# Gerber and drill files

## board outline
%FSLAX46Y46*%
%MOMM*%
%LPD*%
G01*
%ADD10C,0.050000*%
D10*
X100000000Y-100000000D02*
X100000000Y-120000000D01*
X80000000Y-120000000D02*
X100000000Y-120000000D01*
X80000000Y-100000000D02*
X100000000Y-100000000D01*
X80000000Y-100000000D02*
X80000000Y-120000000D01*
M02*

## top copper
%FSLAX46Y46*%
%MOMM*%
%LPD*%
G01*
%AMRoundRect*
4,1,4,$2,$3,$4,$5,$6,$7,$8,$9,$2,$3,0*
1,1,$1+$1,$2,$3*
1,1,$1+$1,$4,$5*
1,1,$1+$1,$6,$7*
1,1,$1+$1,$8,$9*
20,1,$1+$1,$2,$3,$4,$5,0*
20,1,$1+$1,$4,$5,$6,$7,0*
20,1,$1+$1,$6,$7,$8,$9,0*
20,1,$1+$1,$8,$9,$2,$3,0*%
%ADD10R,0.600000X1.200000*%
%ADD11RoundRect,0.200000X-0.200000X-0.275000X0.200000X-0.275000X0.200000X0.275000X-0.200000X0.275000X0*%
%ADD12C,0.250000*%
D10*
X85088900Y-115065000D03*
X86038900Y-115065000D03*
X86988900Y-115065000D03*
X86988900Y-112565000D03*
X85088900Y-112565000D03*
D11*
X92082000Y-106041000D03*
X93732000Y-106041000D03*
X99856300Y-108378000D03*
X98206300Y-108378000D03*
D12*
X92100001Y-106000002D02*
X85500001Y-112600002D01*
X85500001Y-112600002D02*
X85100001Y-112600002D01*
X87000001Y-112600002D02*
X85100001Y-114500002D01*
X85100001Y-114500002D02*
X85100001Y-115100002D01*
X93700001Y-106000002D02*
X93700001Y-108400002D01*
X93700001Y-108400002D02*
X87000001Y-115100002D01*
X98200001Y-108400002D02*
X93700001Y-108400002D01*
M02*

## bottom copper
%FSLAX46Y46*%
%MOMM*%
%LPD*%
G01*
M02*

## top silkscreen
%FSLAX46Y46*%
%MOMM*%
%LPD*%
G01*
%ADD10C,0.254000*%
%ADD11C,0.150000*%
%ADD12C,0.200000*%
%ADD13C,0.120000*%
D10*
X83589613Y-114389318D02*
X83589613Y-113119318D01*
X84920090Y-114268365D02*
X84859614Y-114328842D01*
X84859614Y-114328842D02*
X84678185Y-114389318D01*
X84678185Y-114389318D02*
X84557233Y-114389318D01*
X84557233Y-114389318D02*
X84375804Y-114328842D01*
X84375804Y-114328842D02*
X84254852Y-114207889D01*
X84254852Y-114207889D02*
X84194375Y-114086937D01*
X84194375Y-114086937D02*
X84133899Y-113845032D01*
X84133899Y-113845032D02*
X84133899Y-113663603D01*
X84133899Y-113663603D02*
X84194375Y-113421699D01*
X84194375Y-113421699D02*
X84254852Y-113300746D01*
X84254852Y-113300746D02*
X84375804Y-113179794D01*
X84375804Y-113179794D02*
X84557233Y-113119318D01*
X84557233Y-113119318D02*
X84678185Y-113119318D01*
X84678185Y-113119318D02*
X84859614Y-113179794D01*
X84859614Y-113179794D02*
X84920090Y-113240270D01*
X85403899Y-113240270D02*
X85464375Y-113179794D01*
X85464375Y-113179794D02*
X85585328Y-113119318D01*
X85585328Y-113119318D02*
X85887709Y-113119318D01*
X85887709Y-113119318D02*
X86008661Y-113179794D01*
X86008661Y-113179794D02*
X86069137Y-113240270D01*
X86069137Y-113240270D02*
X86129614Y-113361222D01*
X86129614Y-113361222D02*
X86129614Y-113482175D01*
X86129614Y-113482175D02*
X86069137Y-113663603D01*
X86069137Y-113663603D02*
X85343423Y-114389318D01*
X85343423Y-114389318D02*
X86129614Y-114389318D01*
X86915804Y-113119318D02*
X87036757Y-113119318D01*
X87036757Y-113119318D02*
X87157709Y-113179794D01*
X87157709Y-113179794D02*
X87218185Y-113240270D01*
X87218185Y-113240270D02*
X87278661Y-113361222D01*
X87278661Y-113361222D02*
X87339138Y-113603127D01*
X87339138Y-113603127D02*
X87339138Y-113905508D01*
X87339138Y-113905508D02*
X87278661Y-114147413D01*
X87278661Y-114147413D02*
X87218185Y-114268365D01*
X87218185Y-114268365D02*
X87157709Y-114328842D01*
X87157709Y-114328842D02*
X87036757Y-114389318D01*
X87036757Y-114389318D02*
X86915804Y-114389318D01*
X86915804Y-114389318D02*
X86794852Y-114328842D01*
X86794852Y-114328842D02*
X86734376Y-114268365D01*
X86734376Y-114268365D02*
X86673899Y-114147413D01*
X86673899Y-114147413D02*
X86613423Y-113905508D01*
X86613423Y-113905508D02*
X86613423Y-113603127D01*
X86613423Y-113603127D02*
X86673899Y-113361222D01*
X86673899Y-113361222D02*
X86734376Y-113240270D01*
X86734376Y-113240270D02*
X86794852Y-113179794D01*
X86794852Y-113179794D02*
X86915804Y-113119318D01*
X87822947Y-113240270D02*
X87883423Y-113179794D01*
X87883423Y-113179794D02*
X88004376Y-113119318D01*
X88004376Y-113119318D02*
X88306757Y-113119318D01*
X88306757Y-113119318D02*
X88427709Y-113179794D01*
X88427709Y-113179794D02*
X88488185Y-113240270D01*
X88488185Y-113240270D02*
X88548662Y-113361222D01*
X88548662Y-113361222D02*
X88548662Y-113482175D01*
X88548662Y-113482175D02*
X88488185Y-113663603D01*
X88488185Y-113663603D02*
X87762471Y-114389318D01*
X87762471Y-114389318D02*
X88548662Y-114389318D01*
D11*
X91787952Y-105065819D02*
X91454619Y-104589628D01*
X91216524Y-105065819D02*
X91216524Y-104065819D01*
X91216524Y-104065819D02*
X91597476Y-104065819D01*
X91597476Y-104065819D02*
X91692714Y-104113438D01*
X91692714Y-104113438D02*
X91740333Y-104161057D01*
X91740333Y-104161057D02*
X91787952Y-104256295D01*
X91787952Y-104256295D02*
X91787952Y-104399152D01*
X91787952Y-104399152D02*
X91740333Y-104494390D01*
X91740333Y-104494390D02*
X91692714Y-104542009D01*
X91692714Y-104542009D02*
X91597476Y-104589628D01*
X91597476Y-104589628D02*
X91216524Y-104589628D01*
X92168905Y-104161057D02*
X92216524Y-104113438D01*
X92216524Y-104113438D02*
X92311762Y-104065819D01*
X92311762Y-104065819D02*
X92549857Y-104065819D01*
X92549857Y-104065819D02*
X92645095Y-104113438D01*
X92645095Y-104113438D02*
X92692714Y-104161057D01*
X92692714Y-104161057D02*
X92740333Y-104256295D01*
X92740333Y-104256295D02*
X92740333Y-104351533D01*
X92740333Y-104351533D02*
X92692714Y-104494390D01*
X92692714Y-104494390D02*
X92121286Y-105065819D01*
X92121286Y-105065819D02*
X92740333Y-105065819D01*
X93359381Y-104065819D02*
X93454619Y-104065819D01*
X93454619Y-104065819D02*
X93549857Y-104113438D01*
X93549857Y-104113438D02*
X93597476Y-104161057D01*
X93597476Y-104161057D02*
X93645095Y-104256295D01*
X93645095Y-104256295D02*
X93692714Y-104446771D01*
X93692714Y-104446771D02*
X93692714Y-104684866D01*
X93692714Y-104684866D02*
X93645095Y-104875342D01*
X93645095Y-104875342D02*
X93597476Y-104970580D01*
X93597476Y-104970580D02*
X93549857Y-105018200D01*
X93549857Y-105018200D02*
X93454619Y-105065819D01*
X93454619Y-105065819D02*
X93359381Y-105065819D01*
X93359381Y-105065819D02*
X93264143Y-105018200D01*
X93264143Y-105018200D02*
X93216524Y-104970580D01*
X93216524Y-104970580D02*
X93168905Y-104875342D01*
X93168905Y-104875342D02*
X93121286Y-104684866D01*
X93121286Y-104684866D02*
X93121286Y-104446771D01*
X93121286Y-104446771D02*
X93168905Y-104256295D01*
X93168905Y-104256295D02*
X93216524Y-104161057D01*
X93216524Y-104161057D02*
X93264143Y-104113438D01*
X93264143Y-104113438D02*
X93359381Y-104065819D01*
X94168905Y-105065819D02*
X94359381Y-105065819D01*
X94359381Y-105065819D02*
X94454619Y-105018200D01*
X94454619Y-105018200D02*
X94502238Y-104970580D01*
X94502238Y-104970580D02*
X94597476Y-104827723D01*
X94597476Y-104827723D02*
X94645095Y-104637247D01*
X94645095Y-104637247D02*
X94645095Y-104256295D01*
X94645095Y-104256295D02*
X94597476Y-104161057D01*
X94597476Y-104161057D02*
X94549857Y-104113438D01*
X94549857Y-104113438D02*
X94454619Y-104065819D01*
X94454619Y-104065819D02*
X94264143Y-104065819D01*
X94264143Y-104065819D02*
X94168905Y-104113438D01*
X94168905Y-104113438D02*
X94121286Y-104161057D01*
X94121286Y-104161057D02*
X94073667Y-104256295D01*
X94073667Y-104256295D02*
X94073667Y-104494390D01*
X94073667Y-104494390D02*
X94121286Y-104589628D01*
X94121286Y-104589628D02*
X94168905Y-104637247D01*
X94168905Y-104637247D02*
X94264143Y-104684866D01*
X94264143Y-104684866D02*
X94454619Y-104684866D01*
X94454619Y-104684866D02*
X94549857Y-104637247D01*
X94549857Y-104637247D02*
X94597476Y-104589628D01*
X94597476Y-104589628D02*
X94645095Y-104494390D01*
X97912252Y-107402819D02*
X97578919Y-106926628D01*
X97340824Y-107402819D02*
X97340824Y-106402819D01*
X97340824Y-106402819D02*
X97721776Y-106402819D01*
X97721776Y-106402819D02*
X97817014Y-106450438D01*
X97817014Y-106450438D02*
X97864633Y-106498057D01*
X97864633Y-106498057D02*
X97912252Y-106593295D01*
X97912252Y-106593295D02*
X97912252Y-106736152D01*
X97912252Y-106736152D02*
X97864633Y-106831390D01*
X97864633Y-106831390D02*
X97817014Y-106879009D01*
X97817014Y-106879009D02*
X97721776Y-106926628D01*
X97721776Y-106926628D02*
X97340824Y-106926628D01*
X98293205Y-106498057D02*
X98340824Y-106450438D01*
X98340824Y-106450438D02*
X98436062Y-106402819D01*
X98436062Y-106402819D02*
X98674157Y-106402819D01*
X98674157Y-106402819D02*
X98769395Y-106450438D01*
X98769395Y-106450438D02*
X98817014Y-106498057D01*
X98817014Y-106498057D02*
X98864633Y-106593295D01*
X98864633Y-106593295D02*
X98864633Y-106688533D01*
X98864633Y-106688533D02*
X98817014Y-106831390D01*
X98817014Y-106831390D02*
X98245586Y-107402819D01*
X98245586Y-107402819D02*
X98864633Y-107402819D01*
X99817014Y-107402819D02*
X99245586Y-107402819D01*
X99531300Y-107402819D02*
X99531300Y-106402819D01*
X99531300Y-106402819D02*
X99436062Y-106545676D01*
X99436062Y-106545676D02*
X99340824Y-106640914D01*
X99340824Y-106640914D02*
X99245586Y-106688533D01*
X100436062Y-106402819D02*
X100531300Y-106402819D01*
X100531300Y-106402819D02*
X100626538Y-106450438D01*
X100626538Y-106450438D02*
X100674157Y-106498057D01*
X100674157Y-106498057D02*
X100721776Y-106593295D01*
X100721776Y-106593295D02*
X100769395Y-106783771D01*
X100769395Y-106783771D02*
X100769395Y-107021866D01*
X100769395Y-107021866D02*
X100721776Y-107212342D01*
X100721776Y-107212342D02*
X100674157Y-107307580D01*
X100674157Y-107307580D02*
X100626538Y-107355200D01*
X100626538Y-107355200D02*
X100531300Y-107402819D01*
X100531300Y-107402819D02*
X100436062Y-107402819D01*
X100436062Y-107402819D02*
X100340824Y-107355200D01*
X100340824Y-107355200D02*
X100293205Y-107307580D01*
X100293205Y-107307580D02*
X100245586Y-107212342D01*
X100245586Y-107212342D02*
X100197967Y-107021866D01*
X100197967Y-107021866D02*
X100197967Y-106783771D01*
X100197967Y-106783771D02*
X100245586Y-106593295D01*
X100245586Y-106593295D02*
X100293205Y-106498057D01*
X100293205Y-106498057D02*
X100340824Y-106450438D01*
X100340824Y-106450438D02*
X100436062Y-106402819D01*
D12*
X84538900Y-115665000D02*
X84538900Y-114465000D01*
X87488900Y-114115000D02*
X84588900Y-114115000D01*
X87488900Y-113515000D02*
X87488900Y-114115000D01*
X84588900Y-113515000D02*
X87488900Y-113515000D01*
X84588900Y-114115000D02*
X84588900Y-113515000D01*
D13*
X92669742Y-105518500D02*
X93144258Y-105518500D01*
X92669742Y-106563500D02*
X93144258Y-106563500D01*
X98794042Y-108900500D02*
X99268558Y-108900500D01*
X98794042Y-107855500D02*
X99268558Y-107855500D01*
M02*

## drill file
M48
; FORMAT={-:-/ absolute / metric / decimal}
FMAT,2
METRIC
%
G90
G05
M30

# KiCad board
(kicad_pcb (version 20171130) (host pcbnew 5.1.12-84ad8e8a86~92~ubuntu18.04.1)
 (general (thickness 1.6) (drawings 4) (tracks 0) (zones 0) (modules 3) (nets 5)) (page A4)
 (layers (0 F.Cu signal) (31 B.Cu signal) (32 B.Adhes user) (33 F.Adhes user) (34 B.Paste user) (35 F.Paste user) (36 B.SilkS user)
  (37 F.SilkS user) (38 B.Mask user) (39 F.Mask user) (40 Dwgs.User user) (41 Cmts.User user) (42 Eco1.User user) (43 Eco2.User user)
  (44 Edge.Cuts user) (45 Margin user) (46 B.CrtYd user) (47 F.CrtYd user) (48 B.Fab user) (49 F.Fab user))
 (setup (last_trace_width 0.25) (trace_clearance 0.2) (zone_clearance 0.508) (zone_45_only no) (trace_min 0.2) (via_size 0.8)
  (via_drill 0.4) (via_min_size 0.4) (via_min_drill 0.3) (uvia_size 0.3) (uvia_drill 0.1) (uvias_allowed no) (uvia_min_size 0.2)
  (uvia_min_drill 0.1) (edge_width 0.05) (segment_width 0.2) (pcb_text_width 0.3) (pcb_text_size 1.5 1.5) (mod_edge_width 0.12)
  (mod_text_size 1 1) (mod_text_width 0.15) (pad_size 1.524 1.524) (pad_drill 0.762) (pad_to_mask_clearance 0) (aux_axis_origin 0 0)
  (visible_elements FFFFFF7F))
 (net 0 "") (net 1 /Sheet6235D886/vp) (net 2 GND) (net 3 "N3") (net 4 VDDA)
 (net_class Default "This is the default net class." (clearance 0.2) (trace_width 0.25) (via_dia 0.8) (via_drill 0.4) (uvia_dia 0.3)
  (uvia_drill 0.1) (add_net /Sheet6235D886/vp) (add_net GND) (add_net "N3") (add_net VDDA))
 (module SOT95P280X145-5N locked (layer F.Cu) (at 86.038900 113.815000 90.000000)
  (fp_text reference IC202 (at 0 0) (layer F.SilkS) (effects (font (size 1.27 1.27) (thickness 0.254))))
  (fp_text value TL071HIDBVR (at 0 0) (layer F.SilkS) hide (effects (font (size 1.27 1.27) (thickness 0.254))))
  (fp_line (start -1.85 -1.5) (end -0.65 -1.5) (layer F.SilkS) (width 0.2))
  (fp_line (start -0.3 1.45) (end -0.3 -1.45) (layer F.SilkS) (width 0.2))
  (fp_line (start 0.3 1.45) (end -0.3 1.45) (layer F.SilkS) (width 0.2))
  (fp_line (start 0.3 -1.45) (end 0.3 1.45) (layer F.SilkS) (width 0.2))
  (fp_line (start -0.3 -1.45) (end 0.3 -1.45) (layer F.SilkS) (width 0.2))
  (pad 1 smd rect (at -1.25 -0.95 180.000000) (size 0.6 1.2) (layers F.Cu F.Mask F.Paste) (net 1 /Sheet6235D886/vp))
  (pad 2 smd rect (at -1.25 0 180.000000) (size 0.6 1.2) (layers F.Cu F.Mask F.Paste) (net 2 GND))
  (pad 3 smd rect (at -1.25 0.95 180.000000) (size 0.6 1.2) (layers F.Cu F.Mask F.Paste) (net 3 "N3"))
  (pad 4 smd rect (at 1.25 0.95 180.000000) (size 0.6 1.2) (layers F.Cu F.Mask F.Paste) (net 1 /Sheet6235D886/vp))
  (pad 5 smd rect (at 1.25 -0.95 180.000000) (size 0.6 1.2) (layers F.Cu F.Mask F.Paste) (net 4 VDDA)))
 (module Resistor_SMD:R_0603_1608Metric (layer F.Cu) (at 92.907000 106.041000)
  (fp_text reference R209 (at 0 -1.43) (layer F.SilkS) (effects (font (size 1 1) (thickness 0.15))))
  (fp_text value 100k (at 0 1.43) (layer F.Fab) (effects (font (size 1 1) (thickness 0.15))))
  (fp_line (start -0.237258 -0.5225) (end 0.237258 -0.5225) (layer F.SilkS) (width 0.12))
  (fp_line (start -0.237258 0.5225) (end 0.237258 0.5225) (layer F.SilkS) (width 0.12))
  (pad 1 smd roundrect (at -0.825 0) (size 0.8 0.95) (layers F.Cu F.Mask F.Paste) (roundrect_rratio 0.25) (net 4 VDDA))
  (pad 2 smd roundrect (at 0.825 0) (size 0.8 0.95) (layers F.Cu F.Mask F.Paste) (roundrect_rratio 0.25) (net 3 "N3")))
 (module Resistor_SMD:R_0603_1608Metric (layer F.Cu) (at 99.031300 108.378000)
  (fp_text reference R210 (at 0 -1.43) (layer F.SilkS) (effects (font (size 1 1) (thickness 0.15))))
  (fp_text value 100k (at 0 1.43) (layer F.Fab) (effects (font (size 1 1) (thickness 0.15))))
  (fp_line (start -0.237258 0.5225) (end 0.237258 0.5225) (layer F.SilkS) (width 0.12))
  (fp_line (start -0.237258 -0.5225) (end 0.237258 -0.5225) (layer F.SilkS) (width 0.12))
  (pad 2 smd roundrect (at 0.825 0) (size 0.8 0.95) (layers F.Cu F.Mask F.Paste) (roundrect_rratio 0.25) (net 2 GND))
  (pad 1 smd roundrect (at -0.825 0) (size 0.8 0.95) (layers F.Cu F.Mask F.Paste) (roundrect_rratio 0.25) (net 3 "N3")))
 (gr_line (start 100 100) (end 100 120) (layer Edge.Cuts) (width 0.05))
 (gr_line (start 80 120) (end 100 120) (layer Edge.Cuts) (width 0.05))
 (gr_line (start 80 100) (end 100 100) (layer Edge.Cuts) (width 0.05))
 (gr_line (start 80 100) (end 80 120) (layer Edge.Cuts) (width 0.05))
 (segment (start 92.100001 106.000002) (end 85.500001 112.600002) (width 0.250000) (layer F.Cu) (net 4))
 (segment (start 85.500001 112.600002) (end 85.100001 112.600002) (width 0.250000) (layer F.Cu) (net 4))
 (segment (start 87.000001 112.600002) (end 85.100001 114.500002) (width 0.250000) (layer F.Cu) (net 1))
 (segment (start 85.100001 114.500002) (end 85.100001 115.100002) (width 0.250000) (layer F.Cu) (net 1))
 (segment (start 93.700001 106.000002) (end 93.700001 108.400002) (width 0.250000) (layer F.Cu) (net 3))
 (segment (start 93.700001 108.400002) (end 87.000001 115.100002) (width 0.250000) (layer F.Cu) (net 3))
 (segment (start 98.200001 108.400002) (end 93.700001 108.400002) (width 0.250000) (layer F.Cu) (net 3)))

